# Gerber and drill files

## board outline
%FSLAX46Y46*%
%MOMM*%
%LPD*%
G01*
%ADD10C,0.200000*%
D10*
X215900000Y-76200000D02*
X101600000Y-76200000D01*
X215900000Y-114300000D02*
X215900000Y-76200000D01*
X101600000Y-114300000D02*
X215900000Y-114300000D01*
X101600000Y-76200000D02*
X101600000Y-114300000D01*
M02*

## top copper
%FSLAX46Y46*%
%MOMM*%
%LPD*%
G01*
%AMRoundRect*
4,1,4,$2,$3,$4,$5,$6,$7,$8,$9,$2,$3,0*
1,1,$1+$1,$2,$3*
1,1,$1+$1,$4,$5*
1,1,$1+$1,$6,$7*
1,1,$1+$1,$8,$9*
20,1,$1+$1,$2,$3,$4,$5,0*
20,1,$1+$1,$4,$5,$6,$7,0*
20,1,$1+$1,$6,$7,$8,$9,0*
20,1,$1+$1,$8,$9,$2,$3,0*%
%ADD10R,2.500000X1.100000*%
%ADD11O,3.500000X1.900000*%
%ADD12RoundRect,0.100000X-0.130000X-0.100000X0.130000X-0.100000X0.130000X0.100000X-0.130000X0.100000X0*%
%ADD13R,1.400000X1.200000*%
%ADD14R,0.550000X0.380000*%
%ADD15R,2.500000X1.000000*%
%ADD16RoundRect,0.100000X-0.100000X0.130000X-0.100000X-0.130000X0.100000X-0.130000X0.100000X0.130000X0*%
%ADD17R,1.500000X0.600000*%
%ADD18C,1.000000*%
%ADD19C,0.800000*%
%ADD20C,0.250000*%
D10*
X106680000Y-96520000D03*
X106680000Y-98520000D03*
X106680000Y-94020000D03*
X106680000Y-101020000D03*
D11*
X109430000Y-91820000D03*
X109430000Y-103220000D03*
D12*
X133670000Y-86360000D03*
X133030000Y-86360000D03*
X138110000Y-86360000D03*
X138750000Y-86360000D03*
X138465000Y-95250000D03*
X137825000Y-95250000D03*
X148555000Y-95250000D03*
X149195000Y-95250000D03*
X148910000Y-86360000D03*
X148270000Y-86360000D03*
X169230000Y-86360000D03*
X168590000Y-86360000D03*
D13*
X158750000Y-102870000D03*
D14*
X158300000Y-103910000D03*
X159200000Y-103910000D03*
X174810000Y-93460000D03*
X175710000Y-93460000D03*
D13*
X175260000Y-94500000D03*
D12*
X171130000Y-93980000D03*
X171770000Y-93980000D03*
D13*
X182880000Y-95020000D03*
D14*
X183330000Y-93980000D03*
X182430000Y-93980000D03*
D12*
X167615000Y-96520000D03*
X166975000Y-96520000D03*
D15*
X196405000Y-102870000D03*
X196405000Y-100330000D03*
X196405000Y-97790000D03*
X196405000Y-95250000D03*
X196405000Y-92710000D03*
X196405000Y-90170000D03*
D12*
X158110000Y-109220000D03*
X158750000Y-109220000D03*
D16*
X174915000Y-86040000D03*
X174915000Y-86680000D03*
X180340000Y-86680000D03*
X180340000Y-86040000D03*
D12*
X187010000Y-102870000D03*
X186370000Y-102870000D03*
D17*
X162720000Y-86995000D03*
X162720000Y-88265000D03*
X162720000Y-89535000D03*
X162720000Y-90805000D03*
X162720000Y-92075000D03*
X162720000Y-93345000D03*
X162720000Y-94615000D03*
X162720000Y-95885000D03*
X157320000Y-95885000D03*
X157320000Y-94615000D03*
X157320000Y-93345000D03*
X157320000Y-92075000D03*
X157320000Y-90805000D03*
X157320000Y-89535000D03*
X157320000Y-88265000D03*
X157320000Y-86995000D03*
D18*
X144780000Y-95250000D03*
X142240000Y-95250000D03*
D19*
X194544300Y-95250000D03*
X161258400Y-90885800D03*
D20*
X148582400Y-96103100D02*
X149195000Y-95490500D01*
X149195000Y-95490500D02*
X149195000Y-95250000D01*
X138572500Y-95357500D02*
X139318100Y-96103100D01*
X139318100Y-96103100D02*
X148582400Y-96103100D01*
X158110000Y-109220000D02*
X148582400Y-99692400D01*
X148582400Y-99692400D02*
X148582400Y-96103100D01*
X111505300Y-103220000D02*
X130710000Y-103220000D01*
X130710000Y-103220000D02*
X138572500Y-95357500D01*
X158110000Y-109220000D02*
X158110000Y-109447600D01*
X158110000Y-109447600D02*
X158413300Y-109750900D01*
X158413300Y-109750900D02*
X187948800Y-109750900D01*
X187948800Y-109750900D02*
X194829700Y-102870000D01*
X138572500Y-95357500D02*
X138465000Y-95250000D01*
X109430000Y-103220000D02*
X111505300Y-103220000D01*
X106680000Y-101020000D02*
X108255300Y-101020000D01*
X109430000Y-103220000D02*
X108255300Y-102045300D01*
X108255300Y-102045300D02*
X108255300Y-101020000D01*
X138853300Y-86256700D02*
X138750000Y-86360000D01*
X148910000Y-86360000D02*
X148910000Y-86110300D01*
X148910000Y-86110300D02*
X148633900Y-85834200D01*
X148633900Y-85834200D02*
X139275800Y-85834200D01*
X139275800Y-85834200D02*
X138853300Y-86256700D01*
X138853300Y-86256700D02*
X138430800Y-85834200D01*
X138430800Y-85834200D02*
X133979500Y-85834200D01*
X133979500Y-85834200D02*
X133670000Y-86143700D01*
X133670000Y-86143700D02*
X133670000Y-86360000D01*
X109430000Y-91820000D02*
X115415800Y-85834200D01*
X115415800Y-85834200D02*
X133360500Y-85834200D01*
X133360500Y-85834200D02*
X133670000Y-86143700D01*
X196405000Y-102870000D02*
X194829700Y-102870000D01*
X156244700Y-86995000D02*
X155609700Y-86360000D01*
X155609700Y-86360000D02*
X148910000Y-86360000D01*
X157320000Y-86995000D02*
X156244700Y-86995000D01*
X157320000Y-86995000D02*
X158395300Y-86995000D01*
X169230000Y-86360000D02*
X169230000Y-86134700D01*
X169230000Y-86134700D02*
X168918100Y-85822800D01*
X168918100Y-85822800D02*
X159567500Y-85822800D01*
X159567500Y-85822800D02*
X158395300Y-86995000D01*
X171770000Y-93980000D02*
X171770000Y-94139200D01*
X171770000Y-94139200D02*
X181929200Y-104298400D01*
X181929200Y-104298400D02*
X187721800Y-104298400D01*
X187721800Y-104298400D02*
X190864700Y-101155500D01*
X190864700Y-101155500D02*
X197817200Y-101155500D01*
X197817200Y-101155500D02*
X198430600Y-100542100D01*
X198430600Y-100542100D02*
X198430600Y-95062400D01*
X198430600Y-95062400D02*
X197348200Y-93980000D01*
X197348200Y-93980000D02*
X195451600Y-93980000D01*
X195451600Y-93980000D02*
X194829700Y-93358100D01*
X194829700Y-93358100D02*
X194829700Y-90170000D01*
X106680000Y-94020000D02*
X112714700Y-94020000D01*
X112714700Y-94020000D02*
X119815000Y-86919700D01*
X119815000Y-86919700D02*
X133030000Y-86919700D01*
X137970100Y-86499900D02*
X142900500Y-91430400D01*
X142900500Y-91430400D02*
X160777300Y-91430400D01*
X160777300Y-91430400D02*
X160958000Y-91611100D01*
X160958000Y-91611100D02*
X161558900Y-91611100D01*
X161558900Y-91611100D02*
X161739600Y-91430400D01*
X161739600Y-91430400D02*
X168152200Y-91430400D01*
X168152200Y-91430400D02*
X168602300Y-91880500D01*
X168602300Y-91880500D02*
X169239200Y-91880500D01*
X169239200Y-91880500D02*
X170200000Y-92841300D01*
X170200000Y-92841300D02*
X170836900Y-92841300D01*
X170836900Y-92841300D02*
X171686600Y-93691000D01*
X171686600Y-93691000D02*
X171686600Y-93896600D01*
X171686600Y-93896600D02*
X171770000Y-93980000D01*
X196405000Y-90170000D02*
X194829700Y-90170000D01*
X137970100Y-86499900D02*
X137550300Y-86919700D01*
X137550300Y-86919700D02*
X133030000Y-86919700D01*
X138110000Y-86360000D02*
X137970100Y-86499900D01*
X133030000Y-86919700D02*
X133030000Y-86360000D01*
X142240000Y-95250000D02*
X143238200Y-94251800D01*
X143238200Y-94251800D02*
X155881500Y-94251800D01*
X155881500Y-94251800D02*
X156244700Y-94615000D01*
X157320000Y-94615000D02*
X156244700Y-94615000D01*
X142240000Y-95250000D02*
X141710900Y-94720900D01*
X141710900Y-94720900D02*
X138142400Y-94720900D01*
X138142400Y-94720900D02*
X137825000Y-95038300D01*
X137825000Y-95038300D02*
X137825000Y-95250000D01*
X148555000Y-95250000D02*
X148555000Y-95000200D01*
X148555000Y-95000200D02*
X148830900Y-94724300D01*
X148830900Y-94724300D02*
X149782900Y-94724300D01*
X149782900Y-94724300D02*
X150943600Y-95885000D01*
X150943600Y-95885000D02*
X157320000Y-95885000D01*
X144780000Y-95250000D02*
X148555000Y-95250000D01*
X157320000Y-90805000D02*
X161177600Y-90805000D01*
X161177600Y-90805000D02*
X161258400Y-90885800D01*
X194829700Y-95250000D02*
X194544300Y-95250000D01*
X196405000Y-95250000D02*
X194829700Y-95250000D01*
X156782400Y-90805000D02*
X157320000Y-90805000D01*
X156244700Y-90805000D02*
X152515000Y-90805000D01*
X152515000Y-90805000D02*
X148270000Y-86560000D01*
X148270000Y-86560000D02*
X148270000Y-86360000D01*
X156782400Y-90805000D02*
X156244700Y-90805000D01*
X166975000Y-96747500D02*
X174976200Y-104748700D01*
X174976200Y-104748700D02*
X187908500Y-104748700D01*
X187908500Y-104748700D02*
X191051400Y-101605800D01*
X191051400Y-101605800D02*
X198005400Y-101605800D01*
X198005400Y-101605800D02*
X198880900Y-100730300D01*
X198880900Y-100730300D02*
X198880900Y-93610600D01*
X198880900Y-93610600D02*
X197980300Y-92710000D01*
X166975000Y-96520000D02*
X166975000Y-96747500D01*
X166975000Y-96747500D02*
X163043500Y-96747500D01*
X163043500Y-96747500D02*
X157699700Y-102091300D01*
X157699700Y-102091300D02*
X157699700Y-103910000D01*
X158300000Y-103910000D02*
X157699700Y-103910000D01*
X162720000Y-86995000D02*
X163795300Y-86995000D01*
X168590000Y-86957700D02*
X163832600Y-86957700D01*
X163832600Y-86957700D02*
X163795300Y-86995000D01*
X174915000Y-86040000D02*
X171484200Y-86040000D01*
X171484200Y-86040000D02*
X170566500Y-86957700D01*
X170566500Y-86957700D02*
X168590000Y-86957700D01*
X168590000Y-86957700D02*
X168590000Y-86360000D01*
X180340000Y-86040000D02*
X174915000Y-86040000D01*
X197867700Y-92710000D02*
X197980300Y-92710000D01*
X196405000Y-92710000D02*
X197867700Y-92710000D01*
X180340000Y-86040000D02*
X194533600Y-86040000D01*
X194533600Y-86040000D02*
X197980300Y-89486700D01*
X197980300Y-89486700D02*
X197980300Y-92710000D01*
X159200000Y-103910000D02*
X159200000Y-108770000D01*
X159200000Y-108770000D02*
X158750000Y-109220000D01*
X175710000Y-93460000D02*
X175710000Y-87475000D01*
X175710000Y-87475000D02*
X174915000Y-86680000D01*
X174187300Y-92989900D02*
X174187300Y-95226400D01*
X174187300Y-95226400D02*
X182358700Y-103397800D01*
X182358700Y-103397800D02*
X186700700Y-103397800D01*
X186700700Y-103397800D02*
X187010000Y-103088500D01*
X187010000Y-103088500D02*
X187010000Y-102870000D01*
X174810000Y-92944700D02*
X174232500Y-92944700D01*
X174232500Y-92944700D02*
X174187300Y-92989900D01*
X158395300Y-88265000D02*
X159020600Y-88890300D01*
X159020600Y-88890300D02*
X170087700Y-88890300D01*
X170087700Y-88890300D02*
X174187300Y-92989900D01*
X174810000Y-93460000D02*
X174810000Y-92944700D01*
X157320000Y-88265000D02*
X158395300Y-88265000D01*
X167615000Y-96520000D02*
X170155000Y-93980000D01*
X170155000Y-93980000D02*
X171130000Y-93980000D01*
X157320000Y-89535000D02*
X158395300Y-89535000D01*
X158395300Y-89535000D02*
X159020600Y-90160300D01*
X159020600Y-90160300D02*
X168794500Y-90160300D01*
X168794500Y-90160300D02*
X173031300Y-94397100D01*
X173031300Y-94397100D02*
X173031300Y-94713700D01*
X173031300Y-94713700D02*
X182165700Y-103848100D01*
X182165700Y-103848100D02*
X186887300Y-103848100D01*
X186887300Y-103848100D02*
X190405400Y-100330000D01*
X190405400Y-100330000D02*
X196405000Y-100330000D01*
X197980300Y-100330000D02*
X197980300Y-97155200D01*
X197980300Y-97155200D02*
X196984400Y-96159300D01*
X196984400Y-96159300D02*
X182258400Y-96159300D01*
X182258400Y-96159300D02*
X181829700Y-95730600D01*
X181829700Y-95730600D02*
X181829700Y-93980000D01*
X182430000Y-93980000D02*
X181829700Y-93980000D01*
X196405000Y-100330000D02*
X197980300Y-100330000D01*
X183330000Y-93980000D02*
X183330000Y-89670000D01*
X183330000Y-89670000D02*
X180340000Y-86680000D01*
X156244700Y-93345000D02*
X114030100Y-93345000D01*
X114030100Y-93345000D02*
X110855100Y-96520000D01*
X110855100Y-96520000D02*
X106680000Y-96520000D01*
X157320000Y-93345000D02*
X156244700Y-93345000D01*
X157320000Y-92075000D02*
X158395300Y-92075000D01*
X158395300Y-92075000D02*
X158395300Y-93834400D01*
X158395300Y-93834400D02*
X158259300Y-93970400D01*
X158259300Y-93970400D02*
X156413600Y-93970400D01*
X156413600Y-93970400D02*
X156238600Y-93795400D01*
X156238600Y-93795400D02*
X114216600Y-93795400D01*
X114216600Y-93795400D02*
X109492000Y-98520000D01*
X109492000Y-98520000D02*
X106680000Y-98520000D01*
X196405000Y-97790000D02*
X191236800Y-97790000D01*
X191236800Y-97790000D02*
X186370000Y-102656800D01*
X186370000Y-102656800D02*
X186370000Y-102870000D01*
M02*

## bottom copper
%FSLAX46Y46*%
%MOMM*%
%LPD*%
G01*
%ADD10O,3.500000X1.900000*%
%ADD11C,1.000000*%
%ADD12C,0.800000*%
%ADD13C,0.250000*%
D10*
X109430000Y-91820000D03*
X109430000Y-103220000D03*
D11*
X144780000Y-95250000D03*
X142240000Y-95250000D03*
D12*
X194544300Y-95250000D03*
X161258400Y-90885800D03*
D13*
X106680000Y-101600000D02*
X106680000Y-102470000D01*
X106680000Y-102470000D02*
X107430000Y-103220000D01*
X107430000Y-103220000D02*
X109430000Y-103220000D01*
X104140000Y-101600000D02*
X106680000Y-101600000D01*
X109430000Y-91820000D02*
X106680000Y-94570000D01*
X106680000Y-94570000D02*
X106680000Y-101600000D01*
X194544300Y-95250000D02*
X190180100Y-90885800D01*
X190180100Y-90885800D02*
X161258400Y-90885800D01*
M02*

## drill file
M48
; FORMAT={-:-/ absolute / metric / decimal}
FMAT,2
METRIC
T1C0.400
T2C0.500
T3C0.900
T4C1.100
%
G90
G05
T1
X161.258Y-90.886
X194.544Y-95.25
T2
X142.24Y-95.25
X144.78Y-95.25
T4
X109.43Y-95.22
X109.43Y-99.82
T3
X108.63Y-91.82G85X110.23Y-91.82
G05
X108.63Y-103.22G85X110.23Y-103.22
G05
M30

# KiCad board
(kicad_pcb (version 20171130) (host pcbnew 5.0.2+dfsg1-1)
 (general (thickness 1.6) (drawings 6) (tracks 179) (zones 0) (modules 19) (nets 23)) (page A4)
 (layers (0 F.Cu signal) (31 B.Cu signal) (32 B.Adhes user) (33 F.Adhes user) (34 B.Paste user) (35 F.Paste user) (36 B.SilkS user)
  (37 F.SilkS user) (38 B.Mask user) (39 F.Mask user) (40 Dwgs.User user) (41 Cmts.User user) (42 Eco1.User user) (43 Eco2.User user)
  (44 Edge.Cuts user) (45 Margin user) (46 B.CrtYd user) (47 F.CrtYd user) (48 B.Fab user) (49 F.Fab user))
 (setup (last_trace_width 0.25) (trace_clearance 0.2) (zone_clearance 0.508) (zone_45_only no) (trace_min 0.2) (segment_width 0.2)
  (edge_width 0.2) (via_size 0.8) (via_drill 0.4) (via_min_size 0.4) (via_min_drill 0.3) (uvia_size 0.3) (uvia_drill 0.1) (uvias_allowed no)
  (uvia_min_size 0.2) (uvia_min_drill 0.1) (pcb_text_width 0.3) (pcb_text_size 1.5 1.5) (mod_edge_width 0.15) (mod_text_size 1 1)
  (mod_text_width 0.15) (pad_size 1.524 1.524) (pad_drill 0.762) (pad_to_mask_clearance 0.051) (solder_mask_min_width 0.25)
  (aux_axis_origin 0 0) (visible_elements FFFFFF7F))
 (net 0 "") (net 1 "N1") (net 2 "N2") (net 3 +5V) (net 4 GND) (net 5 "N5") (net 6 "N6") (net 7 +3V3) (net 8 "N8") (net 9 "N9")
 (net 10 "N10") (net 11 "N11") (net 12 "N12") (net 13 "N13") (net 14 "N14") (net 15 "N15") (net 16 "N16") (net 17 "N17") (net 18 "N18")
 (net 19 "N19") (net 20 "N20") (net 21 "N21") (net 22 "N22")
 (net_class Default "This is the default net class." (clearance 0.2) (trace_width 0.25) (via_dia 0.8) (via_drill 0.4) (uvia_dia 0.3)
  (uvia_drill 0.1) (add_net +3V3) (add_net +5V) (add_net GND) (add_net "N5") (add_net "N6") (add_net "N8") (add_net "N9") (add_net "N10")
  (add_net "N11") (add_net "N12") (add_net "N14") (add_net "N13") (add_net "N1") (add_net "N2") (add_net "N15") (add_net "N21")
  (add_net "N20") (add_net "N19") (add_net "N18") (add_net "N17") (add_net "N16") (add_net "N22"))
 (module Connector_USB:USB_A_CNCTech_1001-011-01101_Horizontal (layer F.Cu) (at 116.33 97.52)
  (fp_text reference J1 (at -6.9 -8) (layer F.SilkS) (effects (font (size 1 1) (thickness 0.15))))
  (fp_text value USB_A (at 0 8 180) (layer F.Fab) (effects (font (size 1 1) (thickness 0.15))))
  (pad 2 smd rect (at -9.65 -1) (size 2.5 1.1) (layers F.Cu F.Paste F.Mask) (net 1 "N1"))
  (pad 3 smd rect (at -9.65 1) (size 2.5 1.1) (layers F.Cu F.Paste F.Mask) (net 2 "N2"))
  (pad 1 smd rect (at -9.65 -3.5) (size 2.5 1.1) (layers F.Cu F.Paste F.Mask) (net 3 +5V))
  (pad 4 smd rect (at -9.65 3.5) (size 2.5 1.1) (layers F.Cu F.Paste F.Mask) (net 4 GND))
  (pad 5 thru_hole oval (at -6.9 -5.7) (size 3.5 1.9) (drill oval 2.5 0.9) (layers *.Cu *.Mask) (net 4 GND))
  (pad 5 thru_hole oval (at -6.9 5.7) (size 3.5 1.9) (drill oval 2.5 0.9) (layers *.Cu *.Mask) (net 4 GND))
  (pad "" np_thru_hole circle (at -6.9 -2.3) (size 1.1 1.1) (drill 1.1) (layers *.Cu *.Mask))
  (pad "" np_thru_hole circle (at -6.9 2.3) (size 1.1 1.1) (drill 1.1) (layers *.Cu *.Mask)))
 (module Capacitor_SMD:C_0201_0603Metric (layer F.Cu) (at 133.35 86.36)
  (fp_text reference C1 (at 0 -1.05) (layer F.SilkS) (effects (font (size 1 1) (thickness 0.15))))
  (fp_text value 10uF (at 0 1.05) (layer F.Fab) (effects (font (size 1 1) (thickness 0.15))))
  (pad 2 smd roundrect (at 0.32 0) (size 0.46 0.4) (layers F.Cu F.Mask) (roundrect_rratio 0.25) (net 4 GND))
  (pad 1 smd roundrect (at -0.32 0) (size 0.46 0.4) (layers F.Cu F.Mask) (roundrect_rratio 0.25) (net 3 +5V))
  (pad "" smd roundrect (at 0.345 0) (size 0.318 0.36) (layers F.Paste) (roundrect_rratio 0.25))
  (pad "" smd roundrect (at -0.345 0) (size 0.318 0.36) (layers F.Paste) (roundrect_rratio 0.25)))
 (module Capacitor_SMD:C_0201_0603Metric (layer F.Cu) (at 138.43 86.36)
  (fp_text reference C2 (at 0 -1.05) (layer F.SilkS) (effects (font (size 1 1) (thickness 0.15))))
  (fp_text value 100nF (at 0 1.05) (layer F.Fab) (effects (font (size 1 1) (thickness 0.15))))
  (pad "" smd roundrect (at -0.345 0) (size 0.318 0.36) (layers F.Paste) (roundrect_rratio 0.25))
  (pad "" smd roundrect (at 0.345 0) (size 0.318 0.36) (layers F.Paste) (roundrect_rratio 0.25))
  (pad 1 smd roundrect (at -0.32 0) (size 0.46 0.4) (layers F.Cu F.Mask) (roundrect_rratio 0.25) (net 3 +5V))
  (pad 2 smd roundrect (at 0.32 0) (size 0.46 0.4) (layers F.Cu F.Mask) (roundrect_rratio 0.25) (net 4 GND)))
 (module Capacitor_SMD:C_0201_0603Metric (layer F.Cu) (at 138.145 95.25)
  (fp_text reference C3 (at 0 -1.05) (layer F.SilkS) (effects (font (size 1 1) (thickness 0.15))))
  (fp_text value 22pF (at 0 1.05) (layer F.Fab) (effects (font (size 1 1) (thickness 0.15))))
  (pad 2 smd roundrect (at 0.32 0) (size 0.46 0.4) (layers F.Cu F.Mask) (roundrect_rratio 0.25) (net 4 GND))
  (pad 1 smd roundrect (at -0.32 0) (size 0.46 0.4) (layers F.Cu F.Mask) (roundrect_rratio 0.25) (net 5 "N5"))
  (pad "" smd roundrect (at 0.345 0) (size 0.318 0.36) (layers F.Paste) (roundrect_rratio 0.25))
  (pad "" smd roundrect (at -0.345 0) (size 0.318 0.36) (layers F.Paste) (roundrect_rratio 0.25)))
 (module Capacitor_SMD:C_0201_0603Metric (layer F.Cu) (at 148.875 95.25)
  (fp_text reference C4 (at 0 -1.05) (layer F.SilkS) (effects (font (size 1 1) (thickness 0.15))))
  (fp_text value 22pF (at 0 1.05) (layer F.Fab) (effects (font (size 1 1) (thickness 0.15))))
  (pad "" smd roundrect (at -0.345 0) (size 0.318 0.36) (layers F.Paste) (roundrect_rratio 0.25))
  (pad "" smd roundrect (at 0.345 0) (size 0.318 0.36) (layers F.Paste) (roundrect_rratio 0.25))
  (pad 1 smd roundrect (at -0.32 0) (size 0.46 0.4) (layers F.Cu F.Mask) (roundrect_rratio 0.25) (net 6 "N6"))
  (pad 2 smd roundrect (at 0.32 0) (size 0.46 0.4) (layers F.Cu F.Mask) (roundrect_rratio 0.25) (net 4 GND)))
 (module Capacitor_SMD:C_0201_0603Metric (layer F.Cu) (at 148.59 86.36)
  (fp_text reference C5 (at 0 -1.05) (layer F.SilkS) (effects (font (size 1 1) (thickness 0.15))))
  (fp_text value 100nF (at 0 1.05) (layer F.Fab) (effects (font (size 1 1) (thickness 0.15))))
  (pad 2 smd roundrect (at 0.32 0) (size 0.46 0.4) (layers F.Cu F.Mask) (roundrect_rratio 0.25) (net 4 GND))
  (pad 1 smd roundrect (at -0.32 0) (size 0.46 0.4) (layers F.Cu F.Mask) (roundrect_rratio 0.25) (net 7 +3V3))
  (pad "" smd roundrect (at 0.345 0) (size 0.318 0.36) (layers F.Paste) (roundrect_rratio 0.25))
  (pad "" smd roundrect (at -0.345 0) (size 0.318 0.36) (layers F.Paste) (roundrect_rratio 0.25)))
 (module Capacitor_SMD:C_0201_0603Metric (layer F.Cu) (at 168.91 86.36)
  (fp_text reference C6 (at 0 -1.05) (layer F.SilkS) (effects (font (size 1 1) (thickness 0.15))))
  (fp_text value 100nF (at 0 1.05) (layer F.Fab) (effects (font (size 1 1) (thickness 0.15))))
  (pad 2 smd roundrect (at 0.32 0) (size 0.46 0.4) (layers F.Cu F.Mask) (roundrect_rratio 0.25) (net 4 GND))
  (pad 1 smd roundrect (at -0.32 0) (size 0.46 0.4) (layers F.Cu F.Mask) (roundrect_rratio 0.25) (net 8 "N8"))
  (pad "" smd roundrect (at 0.345 0) (size 0.318 0.36) (layers F.Paste) (roundrect_rratio 0.25))
  (pad "" smd roundrect (at -0.345 0) (size 0.318 0.36) (layers F.Paste) (roundrect_rratio 0.25)))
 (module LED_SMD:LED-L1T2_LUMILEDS (layer F.Cu) (at 158.75 103.39)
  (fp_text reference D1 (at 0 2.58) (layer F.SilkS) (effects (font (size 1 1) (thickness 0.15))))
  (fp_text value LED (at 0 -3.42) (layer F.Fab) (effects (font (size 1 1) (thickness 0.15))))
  (pad 3 smd rect (at 0 -0.52) (size 1.4 1.2) (layers F.Cu F.Paste F.Mask))
  (pad 2 smd rect (at -0.45 0.52) (size 0.55 0.38) (layers F.Cu F.Paste F.Mask) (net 8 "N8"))
  (pad 1 smd rect (at 0.45 0.52) (size 0.55 0.38) (layers F.Cu F.Paste F.Mask) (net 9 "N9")))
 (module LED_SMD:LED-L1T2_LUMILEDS (layer F.Cu) (at 175.26 93.98 180)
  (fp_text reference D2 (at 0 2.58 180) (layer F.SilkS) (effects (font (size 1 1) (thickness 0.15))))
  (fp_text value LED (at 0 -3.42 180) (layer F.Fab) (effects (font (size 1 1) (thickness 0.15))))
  (pad 1 smd rect (at 0.45 0.52 180) (size 0.55 0.38) (layers F.Cu F.Paste F.Mask) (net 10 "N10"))
  (pad 2 smd rect (at -0.45 0.52 180) (size 0.55 0.38) (layers F.Cu F.Paste F.Mask) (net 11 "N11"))
  (pad 3 smd rect (at 0 -0.52 180) (size 1.4 1.2) (layers F.Cu F.Paste F.Mask)))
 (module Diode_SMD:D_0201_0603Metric (layer F.Cu) (at 171.45 93.98)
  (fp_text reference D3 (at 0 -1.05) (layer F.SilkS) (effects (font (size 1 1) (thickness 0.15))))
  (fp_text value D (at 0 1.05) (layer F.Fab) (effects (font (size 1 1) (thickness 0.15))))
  (pad "" smd roundrect (at -0.345 0) (size 0.318 0.36) (layers F.Paste) (roundrect_rratio 0.25))
  (pad "" smd roundrect (at 0.345 0) (size 0.318 0.36) (layers F.Paste) (roundrect_rratio 0.25))
  (pad 1 smd roundrect (at -0.32 0) (size 0.46 0.4) (layers F.Cu F.Mask) (roundrect_rratio 0.25) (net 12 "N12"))
  (pad 2 smd roundrect (at 0.32 0) (size 0.46 0.4) (layers F.Cu F.Mask) (roundrect_rratio 0.25) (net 3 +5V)))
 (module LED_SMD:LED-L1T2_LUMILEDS (layer F.Cu) (at 182.88 94.5 180)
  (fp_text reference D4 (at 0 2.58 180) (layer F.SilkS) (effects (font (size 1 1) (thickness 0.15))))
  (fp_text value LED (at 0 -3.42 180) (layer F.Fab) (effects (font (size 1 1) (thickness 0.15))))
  (pad 3 smd rect (at 0 -0.52 180) (size 1.4 1.2) (layers F.Cu F.Paste F.Mask))
  (pad 2 smd rect (at -0.45 0.52 180) (size 0.55 0.38) (layers F.Cu F.Paste F.Mask) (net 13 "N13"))
  (pad 1 smd rect (at 0.45 0.52 180) (size 0.55 0.38) (layers F.Cu F.Paste F.Mask) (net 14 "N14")))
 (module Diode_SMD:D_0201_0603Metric (layer F.Cu) (at 167.295 96.52)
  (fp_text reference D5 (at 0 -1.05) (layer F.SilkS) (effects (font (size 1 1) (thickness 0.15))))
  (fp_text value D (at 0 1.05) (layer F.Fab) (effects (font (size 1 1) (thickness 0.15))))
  (pad 2 smd roundrect (at 0.32 0) (size 0.46 0.4) (layers F.Cu F.Mask) (roundrect_rratio 0.25) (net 12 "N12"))
  (pad 1 smd roundrect (at -0.32 0) (size 0.46 0.4) (layers F.Cu F.Mask) (roundrect_rratio 0.25) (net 8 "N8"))
  (pad "" smd roundrect (at 0.345 0) (size 0.318 0.36) (layers F.Paste) (roundrect_rratio 0.25))
  (pad "" smd roundrect (at -0.345 0) (size 0.318 0.36) (layers F.Paste) (roundrect_rratio 0.25)))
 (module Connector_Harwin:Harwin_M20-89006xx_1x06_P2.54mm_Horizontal (layer F.Cu) (at 201.93 96.52)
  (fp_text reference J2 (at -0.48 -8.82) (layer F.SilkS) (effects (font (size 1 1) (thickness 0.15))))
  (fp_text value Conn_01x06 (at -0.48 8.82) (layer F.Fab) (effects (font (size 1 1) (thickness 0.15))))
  (pad "" smd rect (at 3.895 -6.35) (size 6 0.76) (layers F.SilkS))
  (pad 6 smd rect (at -5.525 6.35) (size 2.5 1) (layers F.Cu F.Paste F.Mask) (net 4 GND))
  (pad 5 smd rect (at -5.525 3.81) (size 2.5 1) (layers F.Cu F.Paste F.Mask) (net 14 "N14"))
  (pad 4 smd rect (at -5.525 1.27) (size 2.5 1) (layers F.Cu F.Paste F.Mask) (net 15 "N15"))
  (pad 3 smd rect (at -5.525 -1.27) (size 2.5 1) (layers F.Cu F.Paste F.Mask) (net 7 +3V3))
  (pad 2 smd rect (at -5.525 -3.81) (size 2.5 1) (layers F.Cu F.Paste F.Mask) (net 8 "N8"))
  (pad 1 smd rect (at -5.525 -6.35) (size 2.5 1) (layers F.Cu F.Paste F.Mask) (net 3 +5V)))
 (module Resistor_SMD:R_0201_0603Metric (layer F.Cu) (at 158.43 109.22)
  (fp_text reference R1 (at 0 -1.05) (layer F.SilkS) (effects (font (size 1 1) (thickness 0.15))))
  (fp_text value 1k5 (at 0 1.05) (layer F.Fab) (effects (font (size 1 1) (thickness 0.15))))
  (pad "" smd roundrect (at -0.345 0) (size 0.318 0.36) (layers F.Paste) (roundrect_rratio 0.25))
  (pad "" smd roundrect (at 0.345 0) (size 0.318 0.36) (layers F.Paste) (roundrect_rratio 0.25))
  (pad 1 smd roundrect (at -0.32 0) (size 0.46 0.4) (layers F.Cu F.Mask) (roundrect_rratio 0.25) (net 4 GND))
  (pad 2 smd roundrect (at 0.32 0) (size 0.46 0.4) (layers F.Cu F.Mask) (roundrect_rratio 0.25) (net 9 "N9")))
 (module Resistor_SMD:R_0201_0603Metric (layer F.Cu) (at 174.915 86.36 270)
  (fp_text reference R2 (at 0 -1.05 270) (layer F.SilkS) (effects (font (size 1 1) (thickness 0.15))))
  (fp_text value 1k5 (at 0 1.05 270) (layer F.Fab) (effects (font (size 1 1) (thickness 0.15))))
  (pad "" smd roundrect (at -0.345 0 270) (size 0.318 0.36) (layers F.Paste) (roundrect_rratio 0.25))
  (pad "" smd roundrect (at 0.345 0 270) (size 0.318 0.36) (layers F.Paste) (roundrect_rratio 0.25))
  (pad 1 smd roundrect (at -0.32 0 270) (size 0.46 0.4) (layers F.Cu F.Mask) (roundrect_rratio 0.25) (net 8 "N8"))
  (pad 2 smd roundrect (at 0.32 0 270) (size 0.46 0.4) (layers F.Cu F.Mask) (roundrect_rratio 0.25) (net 11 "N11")))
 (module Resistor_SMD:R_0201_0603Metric (layer F.Cu) (at 180.34 86.36 270)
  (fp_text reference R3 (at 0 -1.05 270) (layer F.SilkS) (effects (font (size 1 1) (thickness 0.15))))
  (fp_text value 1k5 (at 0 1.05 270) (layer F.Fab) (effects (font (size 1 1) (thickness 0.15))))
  (pad 2 smd roundrect (at 0.32 0 270) (size 0.46 0.4) (layers F.Cu F.Mask) (roundrect_rratio 0.25) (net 13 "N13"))
  (pad 1 smd roundrect (at -0.32 0 270) (size 0.46 0.4) (layers F.Cu F.Mask) (roundrect_rratio 0.25) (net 8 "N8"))
  (pad "" smd roundrect (at 0.345 0 270) (size 0.318 0.36) (layers F.Paste) (roundrect_rratio 0.25))
  (pad "" smd roundrect (at -0.345 0 270) (size 0.318 0.36) (layers F.Paste) (roundrect_rratio 0.25)))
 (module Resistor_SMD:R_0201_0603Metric (layer F.Cu) (at 186.69 102.87)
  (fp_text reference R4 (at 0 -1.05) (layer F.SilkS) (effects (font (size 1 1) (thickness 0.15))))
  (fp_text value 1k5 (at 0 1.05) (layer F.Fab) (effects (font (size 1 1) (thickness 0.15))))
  (pad 2 smd roundrect (at 0.32 0) (size 0.46 0.4) (layers F.Cu F.Mask) (roundrect_rratio 0.25) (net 10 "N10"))
  (pad 1 smd roundrect (at -0.32 0) (size 0.46 0.4) (layers F.Cu F.Mask) (roundrect_rratio 0.25) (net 15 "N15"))
  (pad "" smd roundrect (at 0.345 0) (size 0.318 0.36) (layers F.Paste) (roundrect_rratio 0.25))
  (pad "" smd roundrect (at -0.345 0) (size 0.318 0.36) (layers F.Paste) (roundrect_rratio 0.25)))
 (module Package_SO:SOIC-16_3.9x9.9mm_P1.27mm (layer F.Cu) (at 160.02 91.44)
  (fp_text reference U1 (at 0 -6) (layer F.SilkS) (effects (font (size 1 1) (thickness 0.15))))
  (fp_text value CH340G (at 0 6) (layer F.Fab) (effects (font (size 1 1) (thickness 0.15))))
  (pad 16 smd rect (at 2.7 -4.445) (size 1.5 0.6) (layers F.Cu F.Paste F.Mask) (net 8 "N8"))
  (pad 15 smd rect (at 2.7 -3.175) (size 1.5 0.6) (layers F.Cu F.Paste F.Mask) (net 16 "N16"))
  (pad 14 smd rect (at 2.7 -1.905) (size 1.5 0.6) (layers F.Cu F.Paste F.Mask) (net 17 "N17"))
  (pad 13 smd rect (at 2.7 -0.635) (size 1.5 0.6) (layers F.Cu F.Paste F.Mask) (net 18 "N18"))
  (pad 12 smd rect (at 2.7 0.635) (size 1.5 0.6) (layers F.Cu F.Paste F.Mask) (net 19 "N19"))
  (pad 11 smd rect (at 2.7 1.905) (size 1.5 0.6) (layers F.Cu F.Paste F.Mask) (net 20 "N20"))
  (pad 10 smd rect (at 2.7 3.175) (size 1.5 0.6) (layers F.Cu F.Paste F.Mask) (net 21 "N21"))
  (pad 9 smd rect (at 2.7 4.445) (size 1.5 0.6) (layers F.Cu F.Paste F.Mask) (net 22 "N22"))
  (pad 8 smd rect (at -2.7 4.445) (size 1.5 0.6) (layers F.Cu F.Paste F.Mask) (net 6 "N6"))
  (pad 7 smd rect (at -2.7 3.175) (size 1.5 0.6) (layers F.Cu F.Paste F.Mask) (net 5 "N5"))
  (pad 6 smd rect (at -2.7 1.905) (size 1.5 0.6) (layers F.Cu F.Paste F.Mask) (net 1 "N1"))
  (pad 5 smd rect (at -2.7 0.635) (size 1.5 0.6) (layers F.Cu F.Paste F.Mask) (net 2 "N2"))
  (pad 4 smd rect (at -2.7 -0.635) (size 1.5 0.6) (layers F.Cu F.Paste F.Mask) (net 7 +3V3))
  (pad 3 smd rect (at -2.7 -1.905) (size 1.5 0.6) (layers F.Cu F.Paste F.Mask) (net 14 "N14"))
  (pad 2 smd rect (at -2.7 -3.175) (size 1.5 0.6) (layers F.Cu F.Paste F.Mask) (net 10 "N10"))
  (pad 1 smd rect (at -2.7 -4.445) (size 1.5 0.6) (layers F.Cu F.Paste F.Mask) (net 4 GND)))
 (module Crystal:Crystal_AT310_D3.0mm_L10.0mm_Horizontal (layer F.Cu) (at 142.24 95.25)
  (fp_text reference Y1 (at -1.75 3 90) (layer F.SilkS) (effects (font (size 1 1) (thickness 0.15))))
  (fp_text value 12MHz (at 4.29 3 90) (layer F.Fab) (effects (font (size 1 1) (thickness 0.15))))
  (pad 2 thru_hole circle (at 2.54 0) (size 1 1) (drill 0.5) (layers *.Cu *.Mask) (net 6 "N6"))
  (pad 1 thru_hole circle (at 0 0) (size 1 1) (drill 0.5) (layers *.Cu *.Mask) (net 5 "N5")))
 (gr_line (start 215.9 76.2) (end 101.6 76.2) (layer Edge.Cuts) (width 0.2))
 (gr_line (start 215.9 114.3) (end 215.9 76.2) (layer Edge.Cuts) (width 0.2))
 (gr_line (start 101.6 114.3) (end 215.9 114.3) (layer Edge.Cuts) (width 0.2))
 (gr_line (start 101.6 76.2) (end 101.6 114.3) (layer Edge.Cuts) (width 0.2))
 (segment (start 148.5824 96.1031) (end 149.195 95.4905) (width 0.25) (layer F.Cu) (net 4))
 (segment (start 149.195 95.4905) (end 149.195 95.25) (width 0.25) (layer F.Cu) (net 4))
 (segment (start 138.5725 95.3575) (end 139.3181 96.1031) (width 0.25) (layer F.Cu) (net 4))
 (segment (start 139.3181 96.1031) (end 148.5824 96.1031) (width 0.25) (layer F.Cu) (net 4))
 (segment (start 158.11 109.22) (end 148.5824 99.6924) (width 0.25) (layer F.Cu) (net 4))
 (segment (start 148.5824 99.6924) (end 148.5824 96.1031) (width 0.25) (layer F.Cu) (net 4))
 (segment (start 111.5053 103.22) (end 130.71 103.22) (width 0.25) (layer F.Cu) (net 4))
 (segment (start 130.71 103.22) (end 138.5725 95.3575) (width 0.25) (layer F.Cu) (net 4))
 (segment (start 158.11 109.22) (end 158.11 109.4476) (width 0.25) (layer F.Cu) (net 4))
 (segment (start 158.11 109.4476) (end 158.4133 109.7509) (width 0.25) (layer F.Cu) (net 4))
 (segment (start 158.4133 109.7509) (end 187.9488 109.7509) (width 0.25) (layer F.Cu) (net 4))
 (segment (start 187.9488 109.7509) (end 194.8297 102.87) (width 0.25) (layer F.Cu) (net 4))
 (segment (start 138.5725 95.3575) (end 138.465 95.25) (width 0.25) (layer F.Cu) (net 4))
 (segment (start 109.43 103.22) (end 111.5053 103.22) (width 0.25) (layer F.Cu) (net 4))
 (segment (start 106.68 101.02) (end 108.2553 101.02) (width 0.25) (layer F.Cu) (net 4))
 (segment (start 109.43 103.22) (end 108.2553 102.0453) (width 0.25) (layer F.Cu) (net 4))
 (segment (start 108.2553 102.0453) (end 108.2553 101.02) (width 0.25) (layer F.Cu) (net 4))
 (segment (start 138.8533 86.2567) (end 138.75 86.36) (width 0.25) (layer F.Cu) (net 4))
 (segment (start 148.91 86.36) (end 148.91 86.1103) (width 0.25) (layer F.Cu) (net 4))
 (segment (start 148.91 86.1103) (end 148.6339 85.8342) (width 0.25) (layer F.Cu) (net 4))
 (segment (start 148.6339 85.8342) (end 139.2758 85.8342) (width 0.25) (layer F.Cu) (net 4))
 (segment (start 139.2758 85.8342) (end 138.8533 86.2567) (width 0.25) (layer F.Cu) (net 4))
 (segment (start 138.8533 86.2567) (end 138.4308 85.8342) (width 0.25) (layer F.Cu) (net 4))
 (segment (start 138.4308 85.8342) (end 133.9795 85.8342) (width 0.25) (layer F.Cu) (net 4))
 (segment (start 133.9795 85.8342) (end 133.67 86.1437) (width 0.25) (layer F.Cu) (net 4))
 (segment (start 133.67 86.1437) (end 133.67 86.36) (width 0.25) (layer F.Cu) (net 4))
 (segment (start 109.43 91.82) (end 115.4158 85.8342) (width 0.25) (layer F.Cu) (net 4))
 (segment (start 115.4158 85.8342) (end 133.3605 85.8342) (width 0.25) (layer F.Cu) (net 4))
 (segment (start 133.3605 85.8342) (end 133.67 86.1437) (width 0.25) (layer F.Cu) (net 4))
 (segment (start 196.405 102.87) (end 194.8297 102.87) (width 0.25) (layer F.Cu) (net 4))
 (segment (start 156.2447 86.995) (end 155.6097 86.36) (width 0.25) (layer F.Cu) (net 4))
 (segment (start 155.6097 86.36) (end 148.91 86.36) (width 0.25) (layer F.Cu) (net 4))
 (segment (start 157.32 86.995) (end 156.2447 86.995) (width 0.25) (layer F.Cu) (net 4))
 (segment (start 106.68 101.6) (end 106.68 102.47) (width 0.25) (layer B.Cu) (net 4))
 (segment (start 106.68 102.47) (end 107.43 103.22) (width 0.25) (layer B.Cu) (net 4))
 (segment (start 107.43 103.22) (end 109.43 103.22) (width 0.25) (layer B.Cu) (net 4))
 (segment (start 104.14 101.6) (end 106.68 101.6) (width 0.25) (layer B.Cu) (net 4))
 (segment (start 109.43 91.82) (end 106.68 94.57) (width 0.25) (layer B.Cu) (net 4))
 (segment (start 106.68 94.57) (end 106.68 101.6) (width 0.25) (layer B.Cu) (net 4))
 (segment (start 157.32 86.995) (end 158.3953 86.995) (width 0.25) (layer F.Cu) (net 4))
 (segment (start 169.23 86.36) (end 169.23 86.1347) (width 0.25) (layer F.Cu) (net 4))
 (segment (start 169.23 86.1347) (end 168.9181 85.8228) (width 0.25) (layer F.Cu) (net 4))
 (segment (start 168.9181 85.8228) (end 159.5675 85.8228) (width 0.25) (layer F.Cu) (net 4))
 (segment (start 159.5675 85.8228) (end 158.3953 86.995) (width 0.25) (layer F.Cu) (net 4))
 (segment (start 171.77 93.98) (end 171.77 94.1392) (width 0.25) (layer F.Cu) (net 3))
 (segment (start 171.77 94.1392) (end 181.9292 104.2984) (width 0.25) (layer F.Cu) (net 3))
 (segment (start 181.9292 104.2984) (end 187.7218 104.2984) (width 0.25) (layer F.Cu) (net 3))
 (segment (start 187.7218 104.2984) (end 190.8647 101.1555) (width 0.25) (layer F.Cu) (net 3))
 (segment (start 190.8647 101.1555) (end 197.8172 101.1555) (width 0.25) (layer F.Cu) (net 3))
 (segment (start 197.8172 101.1555) (end 198.4306 100.5421) (width 0.25) (layer F.Cu) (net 3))
 (segment (start 198.4306 100.5421) (end 198.4306 95.0624) (width 0.25) (layer F.Cu) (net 3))
 (segment (start 198.4306 95.0624) (end 197.3482 93.98) (width 0.25) (layer F.Cu) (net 3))
 (segment (start 197.3482 93.98) (end 195.4516 93.98) (width 0.25) (layer F.Cu) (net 3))
 (segment (start 195.4516 93.98) (end 194.8297 93.3581) (width 0.25) (layer F.Cu) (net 3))
 (segment (start 194.8297 93.3581) (end 194.8297 90.17) (width 0.25) (layer F.Cu) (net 3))
 (segment (start 106.68 94.02) (end 112.7147 94.02) (width 0.25) (layer F.Cu) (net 3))
 (segment (start 112.7147 94.02) (end 119.815 86.9197) (width 0.25) (layer F.Cu) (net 3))
 (segment (start 119.815 86.9197) (end 133.03 86.9197) (width 0.25) (layer F.Cu) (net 3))
 (segment (start 137.9701 86.4999) (end 142.9005 91.4304) (width 0.25) (layer F.Cu) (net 3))
 (segment (start 142.9005 91.4304) (end 160.7773 91.4304) (width 0.25) (layer F.Cu) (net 3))
 (segment (start 160.7773 91.4304) (end 160.958 91.6111) (width 0.25) (layer F.Cu) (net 3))
 (segment (start 160.958 91.6111) (end 161.5589 91.6111) (width 0.25) (layer F.Cu) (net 3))
 (segment (start 161.5589 91.6111) (end 161.7396 91.4304) (width 0.25) (layer F.Cu) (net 3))
 (segment (start 161.7396 91.4304) (end 168.1522 91.4304) (width 0.25) (layer F.Cu) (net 3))
 (segment (start 168.1522 91.4304) (end 168.6023 91.8805) (width 0.25) (layer F.Cu) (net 3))
 (segment (start 168.6023 91.8805) (end 169.2392 91.8805) (width 0.25) (layer F.Cu) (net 3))
 (segment (start 169.2392 91.8805) (end 170.2 92.8413) (width 0.25) (layer F.Cu) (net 3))
 (segment (start 170.2 92.8413) (end 170.8369 92.8413) (width 0.25) (layer F.Cu) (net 3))
 (segment (start 170.8369 92.8413) (end 171.6866 93.691) (width 0.25) (layer F.Cu) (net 3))
 (segment (start 171.6866 93.691) (end 171.6866 93.8966) (width 0.25) (layer F.Cu) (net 3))
 (segment (start 171.6866 93.8966) (end 171.77 93.98) (width 0.25) (layer F.Cu) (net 3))
 (segment (start 196.405 90.17) (end 194.8297 90.17) (width 0.25) (layer F.Cu) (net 3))
 (segment (start 137.9701 86.4999) (end 137.5503 86.9197) (width 0.25) (layer F.Cu) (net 3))
 (segment (start 137.5503 86.9197) (end 133.03 86.9197) (width 0.25) (layer F.Cu) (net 3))
 (segment (start 138.11 86.36) (end 137.9701 86.4999) (width 0.25) (layer F.Cu) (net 3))
 (segment (start 133.03 86.9197) (end 133.03 86.36) (width 0.25) (layer F.Cu) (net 3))
 (segment (start 142.24 95.25) (end 143.2382 94.2518) (width 0.25) (layer F.Cu) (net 5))
 (segment (start 143.2382 94.2518) (end 155.8815 94.2518) (width 0.25) (layer F.Cu) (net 5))
 (segment (start 155.8815 94.2518) (end 156.2447 94.615) (width 0.25) (layer F.Cu) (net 5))
 (segment (start 157.32 94.615) (end 156.2447 94.615) (width 0.25) (layer F.Cu) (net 5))
 (segment (start 142.24 95.25) (end 141.7109 94.7209) (width 0.25) (layer F.Cu) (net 5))
 (segment (start 141.7109 94.7209) (end 138.1424 94.7209) (width 0.25) (layer F.Cu) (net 5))
 (segment (start 138.1424 94.7209) (end 137.825 95.0383) (width 0.25) (layer F.Cu) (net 5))
 (segment (start 137.825 95.0383) (end 137.825 95.25) (width 0.25) (layer F.Cu) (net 5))
 (segment (start 148.555 95.25) (end 148.555 95.0002) (width 0.25) (layer F.Cu) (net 6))
 (segment (start 148.555 95.0002) (end 148.8309 94.7243) (width 0.25) (layer F.Cu) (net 6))
 (segment (start 148.8309 94.7243) (end 149.7829 94.7243) (width 0.25) (layer F.Cu) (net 6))
 (segment (start 149.7829 94.7243) (end 150.9436 95.885) (width 0.25) (layer F.Cu) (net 6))
 (segment (start 150.9436 95.885) (end 157.32 95.885) (width 0.25) (layer F.Cu) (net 6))
 (segment (start 144.78 95.25) (end 148.555 95.25) (width 0.25) (layer F.Cu) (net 6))
 (segment (start 157.32 90.805) (end 161.1776 90.805) (width 0.25) (layer F.Cu) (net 7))
 (segment (start 161.1776 90.805) (end 161.2584 90.8858) (width 0.25) (layer F.Cu) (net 7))
 (segment (start 194.5443 95.25) (end 190.1801 90.8858) (width 0.25) (layer B.Cu) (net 7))
 (segment (start 190.1801 90.8858) (end 161.2584 90.8858) (width 0.25) (layer B.Cu) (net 7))
 (segment (start 194.8297 95.25) (end 194.5443 95.25) (width 0.25) (layer F.Cu) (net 7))
 (segment (start 196.405 95.25) (end 194.8297 95.25) (width 0.25) (layer F.Cu) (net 7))
 (segment (start 156.7824 90.805) (end 157.32 90.805) (width 0.25) (layer F.Cu) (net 7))
 (segment (start 156.2447 90.805) (end 152.515 90.805) (width 0.25) (layer F.Cu) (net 7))
 (segment (start 152.515 90.805) (end 148.27 86.56) (width 0.25) (layer F.Cu) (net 7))
 (segment (start 148.27 86.56) (end 148.27 86.36) (width 0.25) (layer F.Cu) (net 7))
 (segment (start 156.7824 90.805) (end 156.2447 90.805) (width 0.25) (layer F.Cu) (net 7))
 (via (at 194.5443 95.25) (size 0.8) (layers F.Cu B.Cu) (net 7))
 (via (at 161.2584 90.8858) (size 0.8) (layers F.Cu B.Cu) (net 7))
 (segment (start 166.975 96.7475) (end 174.9762 104.7487) (width 0.25) (layer F.Cu) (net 8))
 (segment (start 174.9762 104.7487) (end 187.9085 104.7487) (width 0.25) (layer F.Cu) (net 8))
 (segment (start 187.9085 104.7487) (end 191.0514 101.6058) (width 0.25) (layer F.Cu) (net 8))
 (segment (start 191.0514 101.6058) (end 198.0054 101.6058) (width 0.25) (layer F.Cu) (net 8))
 (segment (start 198.0054 101.6058) (end 198.8809 100.7303) (width 0.25) (layer F.Cu) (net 8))
 (segment (start 198.8809 100.7303) (end 198.8809 93.6106) (width 0.25) (layer F.Cu) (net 8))
 (segment (start 198.8809 93.6106) (end 197.9803 92.71) (width 0.25) (layer F.Cu) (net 8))
 (segment (start 166.975 96.52) (end 166.975 96.7475) (width 0.25) (layer F.Cu) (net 8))
 (segment (start 166.975 96.7475) (end 163.0435 96.7475) (width 0.25) (layer F.Cu) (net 8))
 (segment (start 163.0435 96.7475) (end 157.6997 102.0913) (width 0.25) (layer F.Cu) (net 8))
 (segment (start 157.6997 102.0913) (end 157.6997 103.91) (width 0.25) (layer F.Cu) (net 8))
 (segment (start 158.3 103.91) (end 157.6997 103.91) (width 0.25) (layer F.Cu) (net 8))
 (segment (start 162.72 86.995) (end 163.7953 86.995) (width 0.25) (layer F.Cu) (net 8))
 (segment (start 168.59 86.9577) (end 163.8326 86.9577) (width 0.25) (layer F.Cu) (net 8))
 (segment (start 163.8326 86.9577) (end 163.7953 86.995) (width 0.25) (layer F.Cu) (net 8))
 (segment (start 174.915 86.04) (end 171.4842 86.04) (width 0.25) (layer F.Cu) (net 8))
 (segment (start 171.4842 86.04) (end 170.5665 86.9577) (width 0.25) (layer F.Cu) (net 8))
 (segment (start 170.5665 86.9577) (end 168.59 86.9577) (width 0.25) (layer F.Cu) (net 8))
 (segment (start 168.59 86.9577) (end 168.59 86.36) (width 0.25) (layer F.Cu) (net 8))
 (segment (start 180.34 86.04) (end 174.915 86.04) (width 0.25) (layer F.Cu) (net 8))
 (segment (start 197.8677 92.71) (end 197.9803 92.71) (width 0.25) (layer F.Cu) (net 8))
 (segment (start 196.405 92.71) (end 197.8677 92.71) (width 0.25) (layer F.Cu) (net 8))
 (segment (start 180.34 86.04) (end 194.5336 86.04) (width 0.25) (layer F.Cu) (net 8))
 (segment (start 194.5336 86.04) (end 197.9803 89.4867) (width 0.25) (layer F.Cu) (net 8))
 (segment (start 197.9803 89.4867) (end 197.9803 92.71) (width 0.25) (layer F.Cu) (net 8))
 (segment (start 159.2 103.91) (end 159.2 108.77) (width 0.25) (layer F.Cu) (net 9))
 (segment (start 159.2 108.77) (end 158.75 109.22) (width 0.25) (layer F.Cu) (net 9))
 (segment (start 175.71 93.46) (end 175.71 87.475) (width 0.25) (layer F.Cu) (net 11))
 (segment (start 175.71 87.475) (end 174.915 86.68) (width 0.25) (layer F.Cu) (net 11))
 (segment (start 174.1873 92.9899) (end 174.1873 95.2264) (width 0.25) (layer F.Cu) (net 10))
 (segment (start 174.1873 95.2264) (end 182.3587 103.3978) (width 0.25) (layer F.Cu) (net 10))
 (segment (start 182.3587 103.3978) (end 186.7007 103.3978) (width 0.25) (layer F.Cu) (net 10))
 (segment (start 186.7007 103.3978) (end 187.01 103.0885) (width 0.25) (layer F.Cu) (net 10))
 (segment (start 187.01 103.0885) (end 187.01 102.87) (width 0.25) (layer F.Cu) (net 10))
 (segment (start 174.81 92.9447) (end 174.2325 92.9447) (width 0.25) (layer F.Cu) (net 10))
 (segment (start 174.2325 92.9447) (end 174.1873 92.9899) (width 0.25) (layer F.Cu) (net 10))
 (segment (start 158.3953 88.265) (end 159.0206 88.8903) (width 0.25) (layer F.Cu) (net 10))
 (segment (start 159.0206 88.8903) (end 170.0877 88.8903) (width 0.25) (layer F.Cu) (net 10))
 (segment (start 170.0877 88.8903) (end 174.1873 92.9899) (width 0.25) (layer F.Cu) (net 10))
 (segment (start 174.81 93.46) (end 174.81 92.9447) (width 0.25) (layer F.Cu) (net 10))
 (segment (start 157.32 88.265) (end 158.3953 88.265) (width 0.25) (layer F.Cu) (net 10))
 (segment (start 167.615 96.52) (end 170.155 93.98) (width 0.25) (layer F.Cu) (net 12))
 (segment (start 170.155 93.98) (end 171.13 93.98) (width 0.25) (layer F.Cu) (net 12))
 (segment (start 157.32 89.535) (end 158.3953 89.535) (width 0.25) (layer F.Cu) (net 14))
 (segment (start 158.3953 89.535) (end 159.0206 90.1603) (width 0.25) (layer F.Cu) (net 14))
 (segment (start 159.0206 90.1603) (end 168.7945 90.1603) (width 0.25) (layer F.Cu) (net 14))
 (segment (start 168.7945 90.1603) (end 173.0313 94.3971) (width 0.25) (layer F.Cu) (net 14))
 (segment (start 173.0313 94.3971) (end 173.0313 94.7137) (width 0.25) (layer F.Cu) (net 14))
 (segment (start 173.0313 94.7137) (end 182.1657 103.8481) (width 0.25) (layer F.Cu) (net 14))
 (segment (start 182.1657 103.8481) (end 186.8873 103.8481) (width 0.25) (layer F.Cu) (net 14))
 (segment (start 186.8873 103.8481) (end 190.4054 100.33) (width 0.25) (layer F.Cu) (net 14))
 (segment (start 190.4054 100.33) (end 196.405 100.33) (width 0.25) (layer F.Cu) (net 14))
 (segment (start 197.9803 100.33) (end 197.9803 97.1552) (width 0.25) (layer F.Cu) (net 14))
 (segment (start 197.9803 97.1552) (end 196.9844 96.1593) (width 0.25) (layer F.Cu) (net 14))
 (segment (start 196.9844 96.1593) (end 182.2584 96.1593) (width 0.25) (layer F.Cu) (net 14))
 (segment (start 182.2584 96.1593) (end 181.8297 95.7306) (width 0.25) (layer F.Cu) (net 14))
 (segment (start 181.8297 95.7306) (end 181.8297 93.98) (width 0.25) (layer F.Cu) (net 14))
 (segment (start 182.43 93.98) (end 181.8297 93.98) (width 0.25) (layer F.Cu) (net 14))
 (segment (start 196.405 100.33) (end 197.9803 100.33) (width 0.25) (layer F.Cu) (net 14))
 (segment (start 183.33 93.98) (end 183.33 89.67) (width 0.25) (layer F.Cu) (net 13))
 (segment (start 183.33 89.67) (end 180.34 86.68) (width 0.25) (layer F.Cu) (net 13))
 (segment (start 156.2447 93.345) (end 114.0301 93.345) (width 0.25) (layer F.Cu) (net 1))
 (segment (start 114.0301 93.345) (end 110.8551 96.52) (width 0.25) (layer F.Cu) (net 1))
 (segment (start 110.8551 96.52) (end 106.68 96.52) (width 0.25) (layer F.Cu) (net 1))
 (segment (start 157.32 93.345) (end 156.2447 93.345) (width 0.25) (layer F.Cu) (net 1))
 (segment (start 157.32 92.075) (end 158.3953 92.075) (width 0.25) (layer F.Cu) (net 2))
 (segment (start 158.3953 92.075) (end 158.3953 93.8344) (width 0.25) (layer F.Cu) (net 2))
 (segment (start 158.3953 93.8344) (end 158.2593 93.9704) (width 0.25) (layer F.Cu) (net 2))
 (segment (start 158.2593 93.9704) (end 156.4136 93.9704) (width 0.25) (layer F.Cu) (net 2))
 (segment (start 156.4136 93.9704) (end 156.2386 93.7954) (width 0.25) (layer F.Cu) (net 2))
 (segment (start 156.2386 93.7954) (end 114.2166 93.7954) (width 0.25) (layer F.Cu) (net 2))
 (segment (start 114.2166 93.7954) (end 109.492 98.52) (width 0.25) (layer F.Cu) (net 2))
 (segment (start 109.492 98.52) (end 106.68 98.52) (width 0.25) (layer F.Cu) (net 2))
 (segment (start 196.405 97.79) (end 191.2368 97.79) (width 0.25) (layer F.Cu) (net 15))
 (segment (start 191.2368 97.79) (end 186.37 102.6568) (width 0.25) (layer F.Cu) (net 15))
 (segment (start 186.37 102.6568) (end 186.37 102.87) (width 0.25) (layer F.Cu) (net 15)))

